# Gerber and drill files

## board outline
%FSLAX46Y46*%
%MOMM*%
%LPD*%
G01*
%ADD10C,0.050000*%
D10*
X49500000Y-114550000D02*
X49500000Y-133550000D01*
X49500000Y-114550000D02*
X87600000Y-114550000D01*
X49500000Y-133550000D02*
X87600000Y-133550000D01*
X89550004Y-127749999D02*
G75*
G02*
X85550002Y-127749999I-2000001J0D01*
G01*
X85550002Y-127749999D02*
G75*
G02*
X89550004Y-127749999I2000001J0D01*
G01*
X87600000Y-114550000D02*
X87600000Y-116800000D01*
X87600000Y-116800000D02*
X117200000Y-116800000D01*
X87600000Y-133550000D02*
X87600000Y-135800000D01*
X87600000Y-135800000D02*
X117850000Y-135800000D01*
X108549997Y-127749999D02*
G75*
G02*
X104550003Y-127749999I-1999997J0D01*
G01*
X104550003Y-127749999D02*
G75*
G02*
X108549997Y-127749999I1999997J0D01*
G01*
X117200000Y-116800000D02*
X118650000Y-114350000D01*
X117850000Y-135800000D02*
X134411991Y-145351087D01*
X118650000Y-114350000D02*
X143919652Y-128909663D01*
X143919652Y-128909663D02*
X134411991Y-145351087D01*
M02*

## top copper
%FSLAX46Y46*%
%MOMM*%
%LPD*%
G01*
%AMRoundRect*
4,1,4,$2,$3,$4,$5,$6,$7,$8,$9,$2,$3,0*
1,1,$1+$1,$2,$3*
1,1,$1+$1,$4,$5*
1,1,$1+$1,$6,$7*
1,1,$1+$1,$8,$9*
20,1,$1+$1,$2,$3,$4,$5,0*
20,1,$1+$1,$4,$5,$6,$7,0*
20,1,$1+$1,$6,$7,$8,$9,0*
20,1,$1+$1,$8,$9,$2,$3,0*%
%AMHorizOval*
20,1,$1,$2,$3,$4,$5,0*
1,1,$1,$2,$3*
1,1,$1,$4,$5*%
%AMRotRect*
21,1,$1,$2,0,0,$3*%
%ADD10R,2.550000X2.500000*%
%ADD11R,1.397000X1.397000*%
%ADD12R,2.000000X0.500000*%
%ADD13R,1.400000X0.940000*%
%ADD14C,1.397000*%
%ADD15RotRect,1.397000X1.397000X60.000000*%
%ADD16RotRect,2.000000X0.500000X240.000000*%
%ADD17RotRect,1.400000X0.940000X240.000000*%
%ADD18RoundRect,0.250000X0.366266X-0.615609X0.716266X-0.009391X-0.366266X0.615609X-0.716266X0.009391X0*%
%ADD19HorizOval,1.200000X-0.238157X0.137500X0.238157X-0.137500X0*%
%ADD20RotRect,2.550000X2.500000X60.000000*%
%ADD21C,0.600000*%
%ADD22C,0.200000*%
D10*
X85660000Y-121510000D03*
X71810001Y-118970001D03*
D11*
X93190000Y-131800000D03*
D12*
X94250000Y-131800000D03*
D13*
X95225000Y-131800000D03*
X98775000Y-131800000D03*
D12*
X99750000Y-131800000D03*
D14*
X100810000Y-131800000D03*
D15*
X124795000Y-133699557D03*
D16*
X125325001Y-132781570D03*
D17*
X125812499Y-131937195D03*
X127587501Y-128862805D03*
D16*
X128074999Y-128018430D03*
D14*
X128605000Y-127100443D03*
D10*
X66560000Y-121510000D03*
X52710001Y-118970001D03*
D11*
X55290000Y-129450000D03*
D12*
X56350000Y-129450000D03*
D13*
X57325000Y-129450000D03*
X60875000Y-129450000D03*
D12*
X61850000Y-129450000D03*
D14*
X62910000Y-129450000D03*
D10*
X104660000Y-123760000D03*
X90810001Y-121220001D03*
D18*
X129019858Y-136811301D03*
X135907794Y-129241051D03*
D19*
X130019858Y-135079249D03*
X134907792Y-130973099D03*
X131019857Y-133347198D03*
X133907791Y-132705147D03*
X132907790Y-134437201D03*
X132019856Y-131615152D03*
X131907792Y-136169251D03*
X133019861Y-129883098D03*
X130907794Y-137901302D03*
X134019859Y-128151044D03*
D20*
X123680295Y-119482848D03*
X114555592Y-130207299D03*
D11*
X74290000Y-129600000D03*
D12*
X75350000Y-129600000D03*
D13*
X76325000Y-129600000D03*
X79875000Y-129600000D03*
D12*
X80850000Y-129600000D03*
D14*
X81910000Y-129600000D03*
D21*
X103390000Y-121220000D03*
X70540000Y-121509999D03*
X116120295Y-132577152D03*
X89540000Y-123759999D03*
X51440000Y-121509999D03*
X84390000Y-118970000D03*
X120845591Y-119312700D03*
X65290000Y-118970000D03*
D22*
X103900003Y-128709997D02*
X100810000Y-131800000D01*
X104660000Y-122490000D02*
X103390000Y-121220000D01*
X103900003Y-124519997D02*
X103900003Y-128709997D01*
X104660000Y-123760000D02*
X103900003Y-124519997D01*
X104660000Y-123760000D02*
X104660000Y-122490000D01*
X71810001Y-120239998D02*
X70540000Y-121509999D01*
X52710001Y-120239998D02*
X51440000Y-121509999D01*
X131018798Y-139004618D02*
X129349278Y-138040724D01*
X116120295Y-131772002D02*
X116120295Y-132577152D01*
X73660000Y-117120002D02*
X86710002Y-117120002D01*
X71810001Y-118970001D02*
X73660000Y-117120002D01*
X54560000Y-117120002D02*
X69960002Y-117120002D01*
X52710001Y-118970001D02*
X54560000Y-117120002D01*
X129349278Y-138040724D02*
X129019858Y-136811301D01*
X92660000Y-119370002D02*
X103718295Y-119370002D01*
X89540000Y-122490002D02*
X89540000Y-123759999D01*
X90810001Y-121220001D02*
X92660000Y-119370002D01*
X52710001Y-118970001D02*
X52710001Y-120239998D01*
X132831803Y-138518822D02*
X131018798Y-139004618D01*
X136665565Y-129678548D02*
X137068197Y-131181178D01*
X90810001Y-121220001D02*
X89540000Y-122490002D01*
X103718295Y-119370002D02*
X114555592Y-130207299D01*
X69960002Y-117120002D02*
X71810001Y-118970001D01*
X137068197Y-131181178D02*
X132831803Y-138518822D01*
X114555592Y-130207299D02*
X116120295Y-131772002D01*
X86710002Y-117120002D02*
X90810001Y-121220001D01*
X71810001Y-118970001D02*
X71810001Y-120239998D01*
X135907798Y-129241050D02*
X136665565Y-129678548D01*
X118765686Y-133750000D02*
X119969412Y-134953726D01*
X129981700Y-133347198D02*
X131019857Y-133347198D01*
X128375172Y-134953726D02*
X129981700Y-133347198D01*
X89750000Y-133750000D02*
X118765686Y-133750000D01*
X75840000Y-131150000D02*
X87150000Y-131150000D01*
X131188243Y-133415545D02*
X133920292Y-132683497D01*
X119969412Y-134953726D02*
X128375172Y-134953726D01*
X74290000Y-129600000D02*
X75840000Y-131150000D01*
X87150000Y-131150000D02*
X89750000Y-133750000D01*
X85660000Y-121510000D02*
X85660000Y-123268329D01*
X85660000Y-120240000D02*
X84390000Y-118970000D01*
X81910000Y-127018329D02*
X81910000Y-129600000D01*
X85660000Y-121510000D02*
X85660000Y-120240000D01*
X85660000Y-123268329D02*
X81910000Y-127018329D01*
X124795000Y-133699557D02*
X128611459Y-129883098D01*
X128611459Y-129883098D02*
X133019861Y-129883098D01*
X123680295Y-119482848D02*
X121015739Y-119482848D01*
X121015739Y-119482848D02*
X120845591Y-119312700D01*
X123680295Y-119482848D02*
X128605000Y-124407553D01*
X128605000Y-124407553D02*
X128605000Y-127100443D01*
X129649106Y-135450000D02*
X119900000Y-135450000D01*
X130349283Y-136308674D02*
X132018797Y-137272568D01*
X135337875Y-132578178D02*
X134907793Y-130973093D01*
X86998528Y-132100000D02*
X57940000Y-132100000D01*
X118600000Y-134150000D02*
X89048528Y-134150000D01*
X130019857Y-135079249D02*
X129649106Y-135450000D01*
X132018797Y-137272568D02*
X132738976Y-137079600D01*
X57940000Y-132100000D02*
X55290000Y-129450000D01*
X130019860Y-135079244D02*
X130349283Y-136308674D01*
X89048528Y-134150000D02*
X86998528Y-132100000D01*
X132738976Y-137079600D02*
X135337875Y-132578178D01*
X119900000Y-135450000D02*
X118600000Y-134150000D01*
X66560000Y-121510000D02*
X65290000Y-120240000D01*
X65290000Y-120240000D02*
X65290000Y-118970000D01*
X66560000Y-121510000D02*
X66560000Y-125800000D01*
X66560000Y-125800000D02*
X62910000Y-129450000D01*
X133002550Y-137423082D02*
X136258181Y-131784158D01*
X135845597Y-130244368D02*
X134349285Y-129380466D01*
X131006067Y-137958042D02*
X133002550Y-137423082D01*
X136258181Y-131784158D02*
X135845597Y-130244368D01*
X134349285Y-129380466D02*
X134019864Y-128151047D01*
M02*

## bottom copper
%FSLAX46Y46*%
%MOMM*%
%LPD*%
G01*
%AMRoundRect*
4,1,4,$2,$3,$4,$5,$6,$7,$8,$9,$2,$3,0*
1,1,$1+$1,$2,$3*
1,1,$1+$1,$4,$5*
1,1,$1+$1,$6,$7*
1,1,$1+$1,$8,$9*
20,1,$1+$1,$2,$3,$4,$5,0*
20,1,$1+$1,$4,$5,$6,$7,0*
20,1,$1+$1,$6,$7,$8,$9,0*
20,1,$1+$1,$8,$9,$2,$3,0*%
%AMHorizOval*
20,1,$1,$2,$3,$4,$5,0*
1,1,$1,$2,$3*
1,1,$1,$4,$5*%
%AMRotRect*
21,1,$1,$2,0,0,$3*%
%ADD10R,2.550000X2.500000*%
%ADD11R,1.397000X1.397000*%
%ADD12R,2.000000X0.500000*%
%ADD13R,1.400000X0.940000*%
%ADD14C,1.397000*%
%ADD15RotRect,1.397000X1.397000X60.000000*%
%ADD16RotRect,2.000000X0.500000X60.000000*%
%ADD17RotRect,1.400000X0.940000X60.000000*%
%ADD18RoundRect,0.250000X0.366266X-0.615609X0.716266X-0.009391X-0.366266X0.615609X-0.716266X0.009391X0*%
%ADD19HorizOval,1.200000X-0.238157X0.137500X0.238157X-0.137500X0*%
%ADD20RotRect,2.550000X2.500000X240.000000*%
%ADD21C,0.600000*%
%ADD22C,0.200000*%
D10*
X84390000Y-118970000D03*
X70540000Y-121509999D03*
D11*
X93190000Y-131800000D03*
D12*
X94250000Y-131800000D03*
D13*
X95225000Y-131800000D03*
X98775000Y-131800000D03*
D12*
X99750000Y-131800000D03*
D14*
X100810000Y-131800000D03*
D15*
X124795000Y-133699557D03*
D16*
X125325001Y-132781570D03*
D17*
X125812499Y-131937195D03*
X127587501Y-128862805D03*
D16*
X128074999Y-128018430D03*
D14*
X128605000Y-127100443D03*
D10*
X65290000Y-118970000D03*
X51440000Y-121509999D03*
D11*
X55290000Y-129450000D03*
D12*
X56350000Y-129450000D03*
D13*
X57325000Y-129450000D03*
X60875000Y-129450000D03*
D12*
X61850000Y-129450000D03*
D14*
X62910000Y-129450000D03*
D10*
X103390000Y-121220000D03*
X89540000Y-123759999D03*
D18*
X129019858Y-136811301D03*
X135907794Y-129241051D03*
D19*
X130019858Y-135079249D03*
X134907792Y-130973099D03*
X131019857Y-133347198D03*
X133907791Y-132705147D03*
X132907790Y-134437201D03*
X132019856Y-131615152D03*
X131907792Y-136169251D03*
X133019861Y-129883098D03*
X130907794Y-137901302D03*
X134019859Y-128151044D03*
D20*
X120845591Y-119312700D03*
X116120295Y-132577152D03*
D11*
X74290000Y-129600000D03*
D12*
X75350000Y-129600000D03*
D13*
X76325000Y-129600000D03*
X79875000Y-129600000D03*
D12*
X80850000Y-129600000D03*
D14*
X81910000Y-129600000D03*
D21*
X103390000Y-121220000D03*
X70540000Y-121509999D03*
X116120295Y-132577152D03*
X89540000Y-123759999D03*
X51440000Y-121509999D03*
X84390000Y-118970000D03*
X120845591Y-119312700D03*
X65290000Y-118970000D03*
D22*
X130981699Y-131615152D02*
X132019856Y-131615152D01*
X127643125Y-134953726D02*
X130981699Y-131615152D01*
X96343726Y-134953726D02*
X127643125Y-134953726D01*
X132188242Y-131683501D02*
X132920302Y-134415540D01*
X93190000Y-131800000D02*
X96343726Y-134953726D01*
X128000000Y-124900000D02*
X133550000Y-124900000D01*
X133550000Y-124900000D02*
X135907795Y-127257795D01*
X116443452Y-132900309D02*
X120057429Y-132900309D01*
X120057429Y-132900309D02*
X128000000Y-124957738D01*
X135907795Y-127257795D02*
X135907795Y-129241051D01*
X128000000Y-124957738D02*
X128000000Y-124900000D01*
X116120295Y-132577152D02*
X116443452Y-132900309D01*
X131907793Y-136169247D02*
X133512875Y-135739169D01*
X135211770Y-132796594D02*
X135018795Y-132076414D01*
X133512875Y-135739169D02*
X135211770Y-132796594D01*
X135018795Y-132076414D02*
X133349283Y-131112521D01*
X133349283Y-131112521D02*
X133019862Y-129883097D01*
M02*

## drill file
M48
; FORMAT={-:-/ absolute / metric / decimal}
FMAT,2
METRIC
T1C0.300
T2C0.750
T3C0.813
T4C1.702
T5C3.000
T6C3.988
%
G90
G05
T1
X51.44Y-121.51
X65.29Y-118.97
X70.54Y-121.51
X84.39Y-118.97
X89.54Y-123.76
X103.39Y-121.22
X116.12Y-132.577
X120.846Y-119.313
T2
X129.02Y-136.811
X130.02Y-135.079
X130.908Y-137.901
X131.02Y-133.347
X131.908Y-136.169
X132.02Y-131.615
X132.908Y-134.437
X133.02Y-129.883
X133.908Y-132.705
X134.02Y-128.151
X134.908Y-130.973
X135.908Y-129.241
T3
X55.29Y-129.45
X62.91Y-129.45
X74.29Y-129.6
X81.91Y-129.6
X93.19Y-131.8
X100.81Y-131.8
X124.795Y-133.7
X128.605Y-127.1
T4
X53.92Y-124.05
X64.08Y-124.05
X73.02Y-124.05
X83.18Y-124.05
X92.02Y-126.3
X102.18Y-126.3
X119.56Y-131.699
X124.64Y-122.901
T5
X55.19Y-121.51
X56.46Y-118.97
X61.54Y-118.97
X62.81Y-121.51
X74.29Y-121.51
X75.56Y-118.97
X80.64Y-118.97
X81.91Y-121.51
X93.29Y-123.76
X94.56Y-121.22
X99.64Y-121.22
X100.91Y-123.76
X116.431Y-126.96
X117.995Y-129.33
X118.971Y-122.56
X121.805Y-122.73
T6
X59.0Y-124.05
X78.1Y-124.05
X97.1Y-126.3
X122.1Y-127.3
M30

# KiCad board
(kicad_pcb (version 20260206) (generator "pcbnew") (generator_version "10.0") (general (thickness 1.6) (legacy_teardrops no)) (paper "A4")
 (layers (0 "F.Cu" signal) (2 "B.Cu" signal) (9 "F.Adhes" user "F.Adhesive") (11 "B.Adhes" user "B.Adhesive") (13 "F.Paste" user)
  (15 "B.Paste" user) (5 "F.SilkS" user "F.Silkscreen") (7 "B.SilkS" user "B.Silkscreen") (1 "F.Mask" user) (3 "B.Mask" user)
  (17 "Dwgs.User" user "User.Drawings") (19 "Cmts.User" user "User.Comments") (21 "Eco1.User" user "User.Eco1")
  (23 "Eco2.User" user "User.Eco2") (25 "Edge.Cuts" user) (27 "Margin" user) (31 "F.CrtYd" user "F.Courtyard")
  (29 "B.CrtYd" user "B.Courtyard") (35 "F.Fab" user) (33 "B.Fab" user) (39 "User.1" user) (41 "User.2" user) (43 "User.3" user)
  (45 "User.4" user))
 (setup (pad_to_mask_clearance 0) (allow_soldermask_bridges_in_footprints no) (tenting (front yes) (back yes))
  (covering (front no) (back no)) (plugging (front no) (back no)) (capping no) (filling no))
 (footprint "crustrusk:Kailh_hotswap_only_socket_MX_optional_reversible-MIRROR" (layer "F.Cu") (at 78.1 124.05)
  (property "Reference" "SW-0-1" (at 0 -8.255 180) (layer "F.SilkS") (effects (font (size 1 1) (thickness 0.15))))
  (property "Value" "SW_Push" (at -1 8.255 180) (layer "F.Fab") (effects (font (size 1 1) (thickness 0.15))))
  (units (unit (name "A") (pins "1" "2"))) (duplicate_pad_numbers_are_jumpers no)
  (pad "" np_thru_hole circle (at -5.08 0) (size 1.7018 1.7018) (drill 1.7018) (layers "*.Cu" "*.Mask"))
  (pad "" np_thru_hole circle (at -3.81 -2.54 180) (size 3 3) (drill 3) (layers "*.Cu" "*.Mask"))
  (pad "" np_thru_hole circle (at -2.54 -5.079998) (size 3 3) (drill 3) (layers "*.Cu" "*.Mask"))
  (pad "" np_thru_hole circle (at 0 0) (size 3.9878 3.9878) (drill 3.9878) (layers "*.Cu" "*.Mask"))
  (pad "" np_thru_hole circle (at 2.540002 -5.080001 180) (size 3 3) (drill 3) (layers "*.Cu" "*.Mask"))
  (pad "" np_thru_hole circle (at 3.81 -2.54) (size 3 3) (drill 3) (layers "*.Cu" "*.Mask"))
  (pad "" np_thru_hole circle (at 5.08 0) (size 1.7018 1.7018) (drill 1.7018) (layers "*.Cu" "*.Mask"))
  (pad "1" smd rect (at 6.29 -5.08 180) (size 2.55 2.5) (layers "B.Cu" "B.Mask" "B.Paste") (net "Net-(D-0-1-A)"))
  (pad "1" smd rect (at 7.56 -2.54) (size 2.55 2.5) (layers "F.Cu" "F.Mask" "F.Paste") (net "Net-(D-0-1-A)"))
  (pad "2" smd rect (at -7.56 -2.540001 180) (size 2.55 2.5) (layers "B.Cu" "B.Mask" "B.Paste") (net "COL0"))
  (pad "2" smd rect (at -6.289999 -5.079999) (size 2.55 2.5) (layers "F.Cu" "F.Mask" "F.Paste") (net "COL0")))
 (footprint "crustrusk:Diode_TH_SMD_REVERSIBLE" (layer "F.Cu") (at 97 131.8)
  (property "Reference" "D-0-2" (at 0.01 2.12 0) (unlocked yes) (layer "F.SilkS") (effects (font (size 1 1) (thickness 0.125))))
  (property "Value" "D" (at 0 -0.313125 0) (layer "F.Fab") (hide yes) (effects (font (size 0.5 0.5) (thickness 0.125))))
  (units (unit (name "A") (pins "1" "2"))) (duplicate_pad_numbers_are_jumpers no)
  (pad "1" thru_hole rect (at -3.81 0) (size 1.397 1.397) (drill 0.8128) (layers "*.Cu" "*.Mask") (remove_unused_layers no) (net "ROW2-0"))
  (pad "1" smd rect (at -2.75 0 180) (size 2 0.5) (layers "F.Cu") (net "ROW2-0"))
  (pad "1" smd rect (at -2.75 0) (size 2 0.5) (layers "B.Cu") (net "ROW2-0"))
  (pad "1" smd rect (at -1.775 0 180) (size 1.4 0.94) (layers "F.Cu" "F.Mask" "F.Paste") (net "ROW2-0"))
  (pad "1" smd rect (at -1.775 0) (size 1.4 0.94) (layers "B.Cu" "B.Mask" "B.Paste") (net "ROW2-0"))
  (pad "2" smd rect (at 1.775 0 180) (size 1.4 0.94) (layers "F.Cu" "F.Mask" "F.Paste") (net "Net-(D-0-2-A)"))
  (pad "2" smd rect (at 1.775 0) (size 1.4 0.94) (layers "B.Cu" "B.Mask" "B.Paste") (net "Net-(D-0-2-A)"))
  (pad "2" smd rect (at 2.75 0 180) (size 2 0.5) (layers "F.Cu") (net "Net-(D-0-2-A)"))
  (pad "2" smd rect (at 2.75 0) (size 2 0.5) (layers "B.Cu") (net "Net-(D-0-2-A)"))
  (pad "2" thru_hole circle (at 3.81 0) (size 1.397 1.397) (drill 0.8128) (layers "*.Cu" "*.Mask") (remove_unused_layers no)
   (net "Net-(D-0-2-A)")))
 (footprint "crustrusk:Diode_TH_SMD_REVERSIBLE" (layer "F.Cu") (at 126.7 130.4 60)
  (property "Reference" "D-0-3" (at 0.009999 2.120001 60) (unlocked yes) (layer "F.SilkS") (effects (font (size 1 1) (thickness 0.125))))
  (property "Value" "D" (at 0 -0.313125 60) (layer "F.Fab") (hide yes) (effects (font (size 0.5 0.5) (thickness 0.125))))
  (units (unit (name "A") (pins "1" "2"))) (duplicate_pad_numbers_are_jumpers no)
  (pad "1" thru_hole rect (at -3.81 0 60) (size 1.397 1.397) (drill 0.8128) (layers "*.Cu" "*.Mask") (remove_unused_layers no)
   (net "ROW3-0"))
  (pad "1" smd rect (at -2.75 0.000001 240) (size 2 0.5) (layers "F.Cu") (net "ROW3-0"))
  (pad "1" smd rect (at -2.75 0.000001 60) (size 2 0.5) (layers "B.Cu") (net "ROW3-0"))
  (pad "1" smd rect (at -1.775 -0.000001 240) (size 1.4 0.94) (layers "F.Cu" "F.Mask" "F.Paste") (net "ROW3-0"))
  (pad "1" smd rect (at -1.775 -0.000001 60) (size 1.4 0.94) (layers "B.Cu" "B.Mask" "B.Paste") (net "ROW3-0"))
  (pad "2" smd rect (at 1.775 0.000001 240) (size 1.4 0.94) (layers "F.Cu" "F.Mask" "F.Paste") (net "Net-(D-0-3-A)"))
  (pad "2" smd rect (at 1.775 0.000001 60) (size 1.4 0.94) (layers "B.Cu" "B.Mask" "B.Paste") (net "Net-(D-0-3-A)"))
  (pad "2" smd rect (at 2.75 -0.000001 240) (size 2 0.5) (layers "F.Cu") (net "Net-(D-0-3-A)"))
  (pad "2" smd rect (at 2.75 -0.000001 60) (size 2 0.5) (layers "B.Cu") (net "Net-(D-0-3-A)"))
  (pad "2" thru_hole circle (at 3.81 0 60) (size 1.397 1.397) (drill 0.8128) (layers "*.Cu" "*.Mask") (remove_unused_layers no)
   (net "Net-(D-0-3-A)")))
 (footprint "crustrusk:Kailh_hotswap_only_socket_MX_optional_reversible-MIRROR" (layer "F.Cu") (at 59 124.05)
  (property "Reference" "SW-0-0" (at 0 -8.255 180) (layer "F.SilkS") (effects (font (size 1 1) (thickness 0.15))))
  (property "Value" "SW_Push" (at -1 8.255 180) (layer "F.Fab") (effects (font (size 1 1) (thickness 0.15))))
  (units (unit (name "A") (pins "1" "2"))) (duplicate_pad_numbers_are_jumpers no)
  (pad "" np_thru_hole circle (at -5.08 0) (size 1.7018 1.7018) (drill 1.7018) (layers "*.Cu" "*.Mask"))
  (pad "" np_thru_hole circle (at -3.81 -2.54 180) (size 3 3) (drill 3) (layers "*.Cu" "*.Mask"))
  (pad "" np_thru_hole circle (at -2.54 -5.079998) (size 3 3) (drill 3) (layers "*.Cu" "*.Mask"))
  (pad "" np_thru_hole circle (at 0 0) (size 3.9878 3.9878) (drill 3.9878) (layers "*.Cu" "*.Mask"))
  (pad "" np_thru_hole circle (at 2.540002 -5.080001 180) (size 3 3) (drill 3) (layers "*.Cu" "*.Mask"))
  (pad "" np_thru_hole circle (at 3.81 -2.54) (size 3 3) (drill 3) (layers "*.Cu" "*.Mask"))
  (pad "" np_thru_hole circle (at 5.08 0) (size 1.7018 1.7018) (drill 1.7018) (layers "*.Cu" "*.Mask"))
  (pad "1" smd rect (at 6.29 -5.08 180) (size 2.55 2.5) (layers "B.Cu" "B.Mask" "B.Paste") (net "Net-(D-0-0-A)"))
  (pad "1" smd rect (at 7.56 -2.54) (size 2.55 2.5) (layers "F.Cu" "F.Mask" "F.Paste") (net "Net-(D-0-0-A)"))
  (pad "2" smd rect (at -7.56 -2.540001 180) (size 2.55 2.5) (layers "B.Cu" "B.Mask" "B.Paste") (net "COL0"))
  (pad "2" smd rect (at -6.289999 -5.079999) (size 2.55 2.5) (layers "F.Cu" "F.Mask" "F.Paste") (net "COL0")))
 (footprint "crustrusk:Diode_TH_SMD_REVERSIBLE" (layer "F.Cu") (at 59.1 129.45)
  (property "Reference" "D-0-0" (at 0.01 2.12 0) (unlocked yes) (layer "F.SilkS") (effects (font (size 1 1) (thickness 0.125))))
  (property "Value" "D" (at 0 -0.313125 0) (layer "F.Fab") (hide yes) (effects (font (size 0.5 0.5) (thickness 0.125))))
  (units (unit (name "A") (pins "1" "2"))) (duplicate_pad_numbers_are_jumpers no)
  (pad "1" thru_hole rect (at -3.81 0) (size 1.397 1.397) (drill 0.8128) (layers "*.Cu" "*.Mask") (remove_unused_layers no) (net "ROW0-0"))
  (pad "1" smd rect (at -2.75 0 180) (size 2 0.5) (layers "F.Cu") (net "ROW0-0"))
  (pad "1" smd rect (at -2.75 0) (size 2 0.5) (layers "B.Cu") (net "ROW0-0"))
  (pad "1" smd rect (at -1.775 0 180) (size 1.4 0.94) (layers "F.Cu" "F.Mask" "F.Paste") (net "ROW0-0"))
  (pad "1" smd rect (at -1.775 0) (size 1.4 0.94) (layers "B.Cu" "B.Mask" "B.Paste") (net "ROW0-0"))
  (pad "2" smd rect (at 1.775 0 180) (size 1.4 0.94) (layers "F.Cu" "F.Mask" "F.Paste") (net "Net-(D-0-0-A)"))
  (pad "2" smd rect (at 1.775 0) (size 1.4 0.94) (layers "B.Cu" "B.Mask" "B.Paste") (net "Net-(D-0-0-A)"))
  (pad "2" smd rect (at 2.75 0 180) (size 2 0.5) (layers "F.Cu") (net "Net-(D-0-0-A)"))
  (pad "2" smd rect (at 2.75 0) (size 2 0.5) (layers "B.Cu") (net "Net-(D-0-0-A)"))
  (pad "2" thru_hole circle (at 3.81 0) (size 1.397 1.397) (drill 0.8128) (layers "*.Cu" "*.Mask") (remove_unused_layers no)
   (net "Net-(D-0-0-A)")))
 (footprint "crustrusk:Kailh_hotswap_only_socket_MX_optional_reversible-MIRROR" (layer "F.Cu") (at 97.1 126.3)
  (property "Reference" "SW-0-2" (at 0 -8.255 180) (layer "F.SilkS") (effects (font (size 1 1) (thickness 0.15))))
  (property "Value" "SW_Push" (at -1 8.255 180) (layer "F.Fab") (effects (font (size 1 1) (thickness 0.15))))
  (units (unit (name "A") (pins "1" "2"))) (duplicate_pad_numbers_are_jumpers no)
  (pad "" np_thru_hole circle (at -5.08 0) (size 1.7018 1.7018) (drill 1.7018) (layers "*.Cu" "*.Mask"))
  (pad "" np_thru_hole circle (at -3.81 -2.54 180) (size 3 3) (drill 3) (layers "*.Cu" "*.Mask"))
  (pad "" np_thru_hole circle (at -2.54 -5.079998) (size 3 3) (drill 3) (layers "*.Cu" "*.Mask"))
  (pad "" np_thru_hole circle (at 0 0) (size 3.9878 3.9878) (drill 3.9878) (layers "*.Cu" "*.Mask"))
  (pad "" np_thru_hole circle (at 2.540002 -5.080001 180) (size 3 3) (drill 3) (layers "*.Cu" "*.Mask"))
  (pad "" np_thru_hole circle (at 3.81 -2.54) (size 3 3) (drill 3) (layers "*.Cu" "*.Mask"))
  (pad "" np_thru_hole circle (at 5.08 0) (size 1.7018 1.7018) (drill 1.7018) (layers "*.Cu" "*.Mask"))
  (pad "1" smd rect (at 6.29 -5.08 180) (size 2.55 2.5) (layers "B.Cu" "B.Mask" "B.Paste") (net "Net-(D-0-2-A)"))
  (pad "1" smd rect (at 7.56 -2.54) (size 2.55 2.5) (layers "F.Cu" "F.Mask" "F.Paste") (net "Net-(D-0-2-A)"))
  (pad "2" smd rect (at -7.56 -2.540001 180) (size 2.55 2.5) (layers "B.Cu" "B.Mask" "B.Paste") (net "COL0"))
  (pad "2" smd rect (at -6.289999 -5.079999) (size 2.55 2.5) (layers "F.Cu" "F.Mask" "F.Paste") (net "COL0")))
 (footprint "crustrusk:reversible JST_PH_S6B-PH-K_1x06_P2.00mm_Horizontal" (layer "F.Cu") (at 129.019858 136.811301 60)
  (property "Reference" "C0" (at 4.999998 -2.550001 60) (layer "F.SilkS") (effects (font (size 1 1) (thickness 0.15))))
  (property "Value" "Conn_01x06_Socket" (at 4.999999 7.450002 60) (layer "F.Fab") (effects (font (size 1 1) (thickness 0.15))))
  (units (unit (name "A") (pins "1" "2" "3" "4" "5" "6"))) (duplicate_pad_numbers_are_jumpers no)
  (pad "1" thru_hole roundrect (at 0 0 60) (size 1.2 1.75) (drill 0.75) (layers "*.Cu" "*.Mask") (remove_unused_layers no)
   (roundrect_rratio 0.208333) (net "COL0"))
  (pad "1" thru_hole roundrect (at 9.999997 2.180003 60) (size 1.2 1.75) (drill 0.75) (layers "*.Cu" "*.Mask") (remove_unused_layers no)
   (roundrect_rratio 0.208333) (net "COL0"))
  (pad "2" thru_hole oval (at 2.000001 -0.000001 60) (size 1.2 1.75) (drill 0.75) (layers "*.Cu" "*.Mask") (remove_unused_layers no)
   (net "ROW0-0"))
  (pad "2" thru_hole oval (at 7.999998 2.179999 60) (size 1.2 1.75) (drill 0.75) (layers "*.Cu" "*.Mask") (remove_unused_layers no)
   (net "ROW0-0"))
  (pad "3" thru_hole oval (at 4.000001 -0.000002 60) (size 1.2 1.75) (drill 0.75) (layers "*.Cu" "*.Mask") (remove_unused_layers no)
   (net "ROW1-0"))
  (pad "3" thru_hole oval (at 6 2.179997 60) (size 1.2 1.75) (drill 0.75) (layers "*.Cu" "*.Mask") (remove_unused_layers no) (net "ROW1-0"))
  (pad "4" thru_hole oval (at 3.999997 2.179998 60) (size 1.2 1.75) (drill 0.75) (layers "*.Cu" "*.Mask") (remove_unused_layers no)
   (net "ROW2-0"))
  (pad "4" thru_hole oval (at 5.999996 0 60) (size 1.2 1.75) (drill 0.75) (layers "*.Cu" "*.Mask") (remove_unused_layers no) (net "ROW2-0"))
  (pad "5" thru_hole oval (at 1.999999 2.179999 60) (size 1.2 1.75) (drill 0.75) (layers "*.Cu" "*.Mask") (remove_unused_layers no)
   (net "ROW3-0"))
  (pad "5" thru_hole oval (at 8.000001 0.000003 60) (size 1.2 1.75) (drill 0.75) (layers "*.Cu" "*.Mask") (remove_unused_layers no)
   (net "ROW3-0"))
  (pad "6" thru_hole oval (at 0 2.180001 60) (size 1.2 1.75) (drill 0.75) (layers "*.Cu" "*.Mask") (remove_unused_layers no) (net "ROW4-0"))
  (pad "6" thru_hole oval (at 10.000003 -0.000001 60) (size 1.2 1.75) (drill 0.75) (layers "*.Cu" "*.Mask") (remove_unused_layers no)
   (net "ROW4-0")))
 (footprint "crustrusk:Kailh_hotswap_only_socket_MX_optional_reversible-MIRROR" (layer "F.Cu") (at 122.1 127.3 60)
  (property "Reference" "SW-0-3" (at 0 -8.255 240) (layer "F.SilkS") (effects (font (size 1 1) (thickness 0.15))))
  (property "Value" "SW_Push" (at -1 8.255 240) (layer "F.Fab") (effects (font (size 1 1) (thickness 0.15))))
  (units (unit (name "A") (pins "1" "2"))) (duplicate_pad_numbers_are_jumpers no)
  (pad "" np_thru_hole circle (at -5.08 0 60) (size 1.7018 1.7018) (drill 1.7018) (layers "*.Cu" "*.Mask"))
  (pad "" np_thru_hole circle (at -3.81 -2.54 240) (size 3 3) (drill 3) (layers "*.Cu" "*.Mask"))
  (pad "" np_thru_hole circle (at -2.54 -5.079997 60) (size 3 3) (drill 3) (layers "*.Cu" "*.Mask"))
  (pad "" np_thru_hole circle (at 0 0 60) (size 3.9878 3.9878) (drill 3.9878) (layers "*.Cu" "*.Mask"))
  (pad "" np_thru_hole circle (at 2.540002 -5.080001 240) (size 3 3) (drill 3) (layers "*.Cu" "*.Mask"))
  (pad "" np_thru_hole circle (at 3.81 -2.540001 60) (size 3 3) (drill 3) (layers "*.Cu" "*.Mask"))
  (pad "" np_thru_hole circle (at 5.08 0 60) (size 1.7018 1.7018) (drill 1.7018) (layers "*.Cu" "*.Mask"))
  (pad "1" smd rect (at 6.29 -5.08 240) (size 2.55 2.5) (layers "B.Cu" "B.Mask" "B.Paste") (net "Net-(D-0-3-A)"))
  (pad "1" smd rect (at 7.56 -2.54 60) (size 2.55 2.5) (layers "F.Cu" "F.Mask" "F.Paste") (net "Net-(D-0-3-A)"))
  (pad "2" smd rect (at -7.56 -2.54 240) (size 2.55 2.5) (layers "B.Cu" "B.Mask" "B.Paste") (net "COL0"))
  (pad "2" smd rect (at -6.289999 -5.079999 60) (size 2.55 2.5) (layers "F.Cu" "F.Mask" "F.Paste") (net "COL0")))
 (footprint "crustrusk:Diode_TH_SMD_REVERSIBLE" (layer "F.Cu") (at 78.1 129.6)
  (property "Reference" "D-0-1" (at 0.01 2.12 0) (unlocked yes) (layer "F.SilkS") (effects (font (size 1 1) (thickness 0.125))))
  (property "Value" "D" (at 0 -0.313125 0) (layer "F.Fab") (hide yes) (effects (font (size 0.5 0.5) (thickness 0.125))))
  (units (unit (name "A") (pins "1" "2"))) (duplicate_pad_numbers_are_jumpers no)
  (pad "1" thru_hole rect (at -3.81 0) (size 1.397 1.397) (drill 0.8128) (layers "*.Cu" "*.Mask") (remove_unused_layers no) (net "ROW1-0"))
  (pad "1" smd rect (at -2.75 0 180) (size 2 0.5) (layers "F.Cu") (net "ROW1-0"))
  (pad "1" smd rect (at -2.75 0) (size 2 0.5) (layers "B.Cu") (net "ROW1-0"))
  (pad "1" smd rect (at -1.775 0 180) (size 1.4 0.94) (layers "F.Cu" "F.Mask" "F.Paste") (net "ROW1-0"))
  (pad "1" smd rect (at -1.775 0) (size 1.4 0.94) (layers "B.Cu" "B.Mask" "B.Paste") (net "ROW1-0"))
  (pad "2" smd rect (at 1.775 0 180) (size 1.4 0.94) (layers "F.Cu" "F.Mask" "F.Paste") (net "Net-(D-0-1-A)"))
  (pad "2" smd rect (at 1.775 0) (size 1.4 0.94) (layers "B.Cu" "B.Mask" "B.Paste") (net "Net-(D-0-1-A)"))
  (pad "2" smd rect (at 2.75 0 180) (size 2 0.5) (layers "F.Cu") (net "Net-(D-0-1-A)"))
  (pad "2" smd rect (at 2.75 0) (size 2 0.5) (layers "B.Cu") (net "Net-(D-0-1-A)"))
  (pad "2" thru_hole circle (at 3.81 0) (size 1.397 1.397) (drill 0.8128) (layers "*.Cu" "*.Mask") (remove_unused_layers no)
   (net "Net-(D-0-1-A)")))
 (gr_line (start 49.5 114.55) (end 49.5 133.55) (stroke (width 0.05) (type default)) (layer "Edge.Cuts"))
 (gr_line (start 49.5 114.55) (end 87.6 114.55) (stroke (width 0.05) (type default)) (layer "Edge.Cuts"))
 (gr_line (start 49.5 133.55) (end 87.6 133.55) (stroke (width 0.05) (type default)) (layer "Edge.Cuts"))
 (gr_circle (center 87.550003 127.749999) (end 85.550002 127.749999) (stroke (width 0.05) (type default)) (fill no) (layer "Edge.Cuts"))
 (gr_line (start 87.6 114.55) (end 87.6 116.8) (stroke (width 0.05) (type default)) (layer "Edge.Cuts"))
 (gr_line (start 87.6 116.8) (end 117.2 116.8) (stroke (width 0.05) (type default)) (layer "Edge.Cuts"))
 (gr_line (start 87.6 133.55) (end 87.6 135.8) (stroke (width 0.05) (type default)) (layer "Edge.Cuts"))
 (gr_line (start 87.6 135.8) (end 117.85 135.8) (stroke (width 0.05) (type default)) (layer "Edge.Cuts"))
 (gr_circle (center 106.55 127.749999) (end 104.550003 127.749999) (stroke (width 0.05) (type default)) (fill no) (layer "Edge.Cuts"))
 (gr_line (start 117.2 116.8) (end 118.65 114.35) (stroke (width 0.05) (type default)) (layer "Edge.Cuts"))
 (gr_line (start 117.85 135.8) (end 134.411991 145.351087) (stroke (width 0.05) (type default)) (layer "Edge.Cuts"))
 (gr_line (start 118.65 114.35) (end 143.919652 128.909663) (stroke (width 0.05) (type default)) (layer "Edge.Cuts"))
 (gr_line (start 143.919652 128.909663) (end 134.411991 145.351087) (stroke (width 0.05) (type default)) (layer "Edge.Cuts"))
 (segment (start 130.981699 131.615152) (end 132.019856 131.615152) (width 0.2) (layer "B.Cu") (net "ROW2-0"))
 (segment (start 127.643125 134.953726) (end 130.981699 131.615152) (width 0.2) (layer "B.Cu") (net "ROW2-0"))
 (segment (start 96.343726 134.953726) (end 127.643125 134.953726) (width 0.2) (layer "B.Cu") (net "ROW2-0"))
 (segment (start 132.188242 131.683501) (end 132.920302 134.41554) (width 0.2) (layer "B.Cu") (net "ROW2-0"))
 (segment (start 93.19 131.8) (end 96.343726 134.953726) (width 0.2) (layer "B.Cu") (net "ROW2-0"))
 (segment (start 103.900003 128.709997) (end 100.81 131.8) (width 0.2) (layer "F.Cu") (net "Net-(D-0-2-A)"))
 (segment (start 104.66 122.49) (end 103.39 121.22) (width 0.2) (layer "F.Cu") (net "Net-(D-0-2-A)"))
 (segment (start 103.900003 124.519997) (end 103.900003 128.709997) (width 0.2) (layer "F.Cu") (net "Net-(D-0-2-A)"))
 (segment (start 104.66 123.76) (end 103.900003 124.519997) (width 0.2) (layer "F.Cu") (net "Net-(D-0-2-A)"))
 (segment (start 104.66 123.76) (end 104.66 122.49) (width 0.2) (layer "F.Cu") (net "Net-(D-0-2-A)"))
 (via (at 103.39 121.22) (size 0.6) (drill 0.3) (layers "F.Cu" "B.Cu") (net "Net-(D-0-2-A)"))
 (segment (start 71.810001 120.239998) (end 70.54 121.509999) (width 0.2) (layer "F.Cu") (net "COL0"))
 (segment (start 52.710001 120.239998) (end 51.44 121.509999) (width 0.2) (layer "F.Cu") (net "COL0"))
 (segment (start 131.018798 139.004618) (end 129.349278 138.040724) (width 0.2) (layer "F.Cu") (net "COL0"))
 (segment (start 116.120295 131.772002) (end 116.120295 132.577152) (width 0.2) (layer "F.Cu") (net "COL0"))
 (segment (start 73.66 117.120002) (end 86.710002 117.120002) (width 0.2) (layer "F.Cu") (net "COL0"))
 (segment (start 71.810001 118.970001) (end 73.66 117.120002) (width 0.2) (layer "F.Cu") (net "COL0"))
 (segment (start 54.56 117.120002) (end 69.960002 117.120002) (width 0.2) (layer "F.Cu") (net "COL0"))
 (segment (start 52.710001 118.970001) (end 54.56 117.120002) (width 0.2) (layer "F.Cu") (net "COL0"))
 (segment (start 129.349278 138.040724) (end 129.019858 136.811301) (width 0.2) (layer "F.Cu") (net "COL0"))
 (segment (start 92.66 119.370002) (end 103.718295 119.370002) (width 0.2) (layer "F.Cu") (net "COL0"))
 (segment (start 89.54 122.490002) (end 89.54 123.759999) (width 0.2) (layer "F.Cu") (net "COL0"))
 (segment (start 90.810001 121.220001) (end 92.66 119.370002) (width 0.2) (layer "F.Cu") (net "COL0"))
 (segment (start 52.710001 118.970001) (end 52.710001 120.239998) (width 0.2) (layer "F.Cu") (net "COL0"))
 (segment (start 132.831803 138.518822) (end 131.018798 139.004618) (width 0.2) (layer "F.Cu") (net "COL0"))
 (segment (start 136.665565 129.678548) (end 137.068197 131.181178) (width 0.2) (layer "F.Cu") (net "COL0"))
 (segment (start 90.810001 121.220001) (end 89.54 122.490002) (width 0.2) (layer "F.Cu") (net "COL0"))
 (segment (start 103.718295 119.370002) (end 114.555592 130.207299) (width 0.2) (layer "F.Cu") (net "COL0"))
 (segment (start 69.960002 117.120002) (end 71.810001 118.970001) (width 0.2) (layer "F.Cu") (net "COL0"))
 (segment (start 137.068197 131.181178) (end 132.831803 138.518822) (width 0.2) (layer "F.Cu") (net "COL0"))
 (segment (start 114.555592 130.207299) (end 116.120295 131.772002) (width 0.2) (layer "F.Cu") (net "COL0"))
 (segment (start 86.710002 117.120002) (end 90.810001 121.220001) (width 0.2) (layer "F.Cu") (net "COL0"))
 (segment (start 71.810001 118.970001) (end 71.810001 120.239998) (width 0.2) (layer "F.Cu") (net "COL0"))
 (segment (start 135.907798 129.24105) (end 136.665565 129.678548) (width 0.2) (layer "F.Cu") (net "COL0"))
 (via (at 70.54 121.509999) (size 0.6) (drill 0.3) (layers "F.Cu" "B.Cu") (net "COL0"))
 (via (at 116.120295 132.577152) (size 0.6) (drill 0.3) (layers "F.Cu" "B.Cu") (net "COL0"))
 (via (at 89.54 123.759999) (size 0.6) (drill 0.3) (layers "F.Cu" "B.Cu") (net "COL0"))
 (via (at 51.44 121.509999) (size 0.6) (drill 0.3) (layers "F.Cu" "B.Cu") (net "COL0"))
 (segment (start 128 124.9) (end 133.55 124.9) (width 0.2) (layer "B.Cu") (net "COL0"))
 (segment (start 133.55 124.9) (end 135.907795 127.257795) (width 0.2) (layer "B.Cu") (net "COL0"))
 (segment (start 116.443452 132.900309) (end 120.057429 132.900309) (width 0.2) (layer "B.Cu") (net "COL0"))
 (segment (start 120.057429 132.900309) (end 128 124.957738) (width 0.2) (layer "B.Cu") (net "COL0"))
 (segment (start 135.907795 127.257795) (end 135.907795 129.241051) (width 0.2) (layer "B.Cu") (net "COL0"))
 (segment (start 128 124.957738) (end 128 124.9) (width 0.2) (layer "B.Cu") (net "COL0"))
 (segment (start 116.120295 132.577152) (end 116.443452 132.900309) (width 0.2) (layer "B.Cu") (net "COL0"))
 (segment (start 118.765686 133.75) (end 119.969412 134.953726) (width 0.2) (layer "F.Cu") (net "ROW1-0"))
 (segment (start 129.9817 133.347198) (end 131.019857 133.347198) (width 0.2) (layer "F.Cu") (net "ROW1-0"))
 (segment (start 128.375172 134.953726) (end 129.9817 133.347198) (width 0.2) (layer "F.Cu") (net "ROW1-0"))
 (segment (start 89.75 133.75) (end 118.765686 133.75) (width 0.2) (layer "F.Cu") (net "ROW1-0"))
 (segment (start 75.84 131.15) (end 87.15 131.15) (width 0.2) (layer "F.Cu") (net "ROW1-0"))
 (segment (start 131.188243 133.415545) (end 133.920292 132.683497) (width 0.2) (layer "F.Cu") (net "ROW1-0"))
 (segment (start 119.969412 134.953726) (end 128.375172 134.953726) (width 0.2) (layer "F.Cu") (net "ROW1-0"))
 (segment (start 74.29 129.6) (end 75.84 131.15) (width 0.2) (layer "F.Cu") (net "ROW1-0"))
 (segment (start 87.15 131.15) (end 89.75 133.75) (width 0.2) (layer "F.Cu") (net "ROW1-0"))
 (segment (start 85.66 121.51) (end 85.66 123.268329) (width 0.2) (layer "F.Cu") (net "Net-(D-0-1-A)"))
 (segment (start 85.66 120.24) (end 84.39 118.97) (width 0.2) (layer "F.Cu") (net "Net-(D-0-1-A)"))
 (segment (start 81.91 127.018329) (end 81.91 129.6) (width 0.2) (layer "F.Cu") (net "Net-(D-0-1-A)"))
 (segment (start 85.66 121.51) (end 85.66 120.24) (width 0.2) (layer "F.Cu") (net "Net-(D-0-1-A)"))
 (segment (start 85.66 123.268329) (end 81.91 127.018329) (width 0.2) (layer "F.Cu") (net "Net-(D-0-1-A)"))
 (via (at 84.39 118.97) (size 0.6) (drill 0.3) (layers "F.Cu" "B.Cu") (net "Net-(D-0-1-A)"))
 (segment (start 124.795 133.699557) (end 128.611459 129.883098) (width 0.2) (layer "F.Cu") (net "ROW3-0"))
 (segment (start 128.611459 129.883098) (end 133.019861 129.883098) (width 0.2) (layer "F.Cu") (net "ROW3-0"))
 (segment (start 131.907793 136.169247) (end 133.512875 135.739169) (width 0.2) (layer "B.Cu") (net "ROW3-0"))
 (segment (start 135.21177 132.796594) (end 135.018795 132.076414) (width 0.2) (layer "B.Cu") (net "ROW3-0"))
 (segment (start 133.512875 135.739169) (end 135.21177 132.796594) (width 0.2) (layer "B.Cu") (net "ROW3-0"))
 (segment (start 135.018795 132.076414) (end 133.349283 131.112521) (width 0.2) (layer "B.Cu") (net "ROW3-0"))
 (segment (start 133.349283 131.112521) (end 133.019862 129.883097) (width 0.2) (layer "B.Cu") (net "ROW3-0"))
 (segment (start 123.680295 119.482848) (end 121.015739 119.482848) (width 0.2) (layer "F.Cu") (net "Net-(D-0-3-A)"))
 (segment (start 121.015739 119.482848) (end 120.845591 119.3127) (width 0.2) (layer "F.Cu") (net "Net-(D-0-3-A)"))
 (segment (start 123.680295 119.482848) (end 128.605 124.407553) (width 0.2) (layer "F.Cu") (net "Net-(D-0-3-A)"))
 (segment (start 128.605 124.407553) (end 128.605 127.100443) (width 0.2) (layer "F.Cu") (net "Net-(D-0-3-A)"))
 (via (at 120.845591 119.3127) (size 0.6) (drill 0.3) (layers "F.Cu" "B.Cu") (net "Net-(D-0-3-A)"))
 (segment (start 129.649106 135.45) (end 119.9 135.45) (width 0.2) (layer "F.Cu") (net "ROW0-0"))
 (segment (start 130.349283 136.308674) (end 132.018797 137.272568) (width 0.2) (layer "F.Cu") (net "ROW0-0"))
 (segment (start 135.337875 132.578178) (end 134.907793 130.973093) (width 0.2) (layer "F.Cu") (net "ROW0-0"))
 (segment (start 86.998528 132.1) (end 57.94 132.1) (width 0.2) (layer "F.Cu") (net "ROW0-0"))
 (segment (start 118.6 134.15) (end 89.048528 134.15) (width 0.2) (layer "F.Cu") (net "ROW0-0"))
 (segment (start 130.019857 135.079249) (end 129.649106 135.45) (width 0.2) (layer "F.Cu") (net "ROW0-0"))
 (segment (start 132.018797 137.272568) (end 132.738976 137.0796) (width 0.2) (layer "F.Cu") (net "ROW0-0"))
 (segment (start 57.94 132.1) (end 55.29 129.45) (width 0.2) (layer "F.Cu") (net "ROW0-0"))
 (segment (start 130.01986 135.079244) (end 130.349283 136.308674) (width 0.2) (layer "F.Cu") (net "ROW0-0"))
 (segment (start 89.048528 134.15) (end 86.998528 132.1) (width 0.2) (layer "F.Cu") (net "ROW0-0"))
 (segment (start 132.738976 137.0796) (end 135.337875 132.578178) (width 0.2) (layer "F.Cu") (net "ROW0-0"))
 (segment (start 119.9 135.45) (end 118.6 134.15) (width 0.2) (layer "F.Cu") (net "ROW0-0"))
 (segment (start 66.56 121.51) (end 65.29 120.24) (width 0.2) (layer "F.Cu") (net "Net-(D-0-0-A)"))
 (segment (start 65.29 120.24) (end 65.29 118.97) (width 0.2) (layer "F.Cu") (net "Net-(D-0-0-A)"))
 (segment (start 66.56 121.51) (end 66.56 125.8) (width 0.2) (layer "F.Cu") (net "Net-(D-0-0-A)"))
 (segment (start 66.56 125.8) (end 62.91 129.45) (width 0.2) (layer "F.Cu") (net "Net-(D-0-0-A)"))
 (via (at 65.29 118.97) (size 0.6) (drill 0.3) (layers "F.Cu" "B.Cu") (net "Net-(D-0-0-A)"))
 (segment (start 133.00255 137.423082) (end 136.258181 131.784158) (width 0.2) (layer "F.Cu") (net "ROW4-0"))
 (segment (start 135.845597 130.244368) (end 134.349285 129.380466) (width 0.2) (layer "F.Cu") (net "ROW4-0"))
 (segment (start 131.006067 137.958042) (end 133.00255 137.423082) (width 0.2) (layer "F.Cu") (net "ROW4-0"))
 (segment (start 136.258181 131.784158) (end 135.845597 130.244368) (width 0.2) (layer "F.Cu") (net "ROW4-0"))
 (segment (start 134.349285 129.380466) (end 134.019864 128.151047) (width 0.2) (layer "F.Cu") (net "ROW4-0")))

